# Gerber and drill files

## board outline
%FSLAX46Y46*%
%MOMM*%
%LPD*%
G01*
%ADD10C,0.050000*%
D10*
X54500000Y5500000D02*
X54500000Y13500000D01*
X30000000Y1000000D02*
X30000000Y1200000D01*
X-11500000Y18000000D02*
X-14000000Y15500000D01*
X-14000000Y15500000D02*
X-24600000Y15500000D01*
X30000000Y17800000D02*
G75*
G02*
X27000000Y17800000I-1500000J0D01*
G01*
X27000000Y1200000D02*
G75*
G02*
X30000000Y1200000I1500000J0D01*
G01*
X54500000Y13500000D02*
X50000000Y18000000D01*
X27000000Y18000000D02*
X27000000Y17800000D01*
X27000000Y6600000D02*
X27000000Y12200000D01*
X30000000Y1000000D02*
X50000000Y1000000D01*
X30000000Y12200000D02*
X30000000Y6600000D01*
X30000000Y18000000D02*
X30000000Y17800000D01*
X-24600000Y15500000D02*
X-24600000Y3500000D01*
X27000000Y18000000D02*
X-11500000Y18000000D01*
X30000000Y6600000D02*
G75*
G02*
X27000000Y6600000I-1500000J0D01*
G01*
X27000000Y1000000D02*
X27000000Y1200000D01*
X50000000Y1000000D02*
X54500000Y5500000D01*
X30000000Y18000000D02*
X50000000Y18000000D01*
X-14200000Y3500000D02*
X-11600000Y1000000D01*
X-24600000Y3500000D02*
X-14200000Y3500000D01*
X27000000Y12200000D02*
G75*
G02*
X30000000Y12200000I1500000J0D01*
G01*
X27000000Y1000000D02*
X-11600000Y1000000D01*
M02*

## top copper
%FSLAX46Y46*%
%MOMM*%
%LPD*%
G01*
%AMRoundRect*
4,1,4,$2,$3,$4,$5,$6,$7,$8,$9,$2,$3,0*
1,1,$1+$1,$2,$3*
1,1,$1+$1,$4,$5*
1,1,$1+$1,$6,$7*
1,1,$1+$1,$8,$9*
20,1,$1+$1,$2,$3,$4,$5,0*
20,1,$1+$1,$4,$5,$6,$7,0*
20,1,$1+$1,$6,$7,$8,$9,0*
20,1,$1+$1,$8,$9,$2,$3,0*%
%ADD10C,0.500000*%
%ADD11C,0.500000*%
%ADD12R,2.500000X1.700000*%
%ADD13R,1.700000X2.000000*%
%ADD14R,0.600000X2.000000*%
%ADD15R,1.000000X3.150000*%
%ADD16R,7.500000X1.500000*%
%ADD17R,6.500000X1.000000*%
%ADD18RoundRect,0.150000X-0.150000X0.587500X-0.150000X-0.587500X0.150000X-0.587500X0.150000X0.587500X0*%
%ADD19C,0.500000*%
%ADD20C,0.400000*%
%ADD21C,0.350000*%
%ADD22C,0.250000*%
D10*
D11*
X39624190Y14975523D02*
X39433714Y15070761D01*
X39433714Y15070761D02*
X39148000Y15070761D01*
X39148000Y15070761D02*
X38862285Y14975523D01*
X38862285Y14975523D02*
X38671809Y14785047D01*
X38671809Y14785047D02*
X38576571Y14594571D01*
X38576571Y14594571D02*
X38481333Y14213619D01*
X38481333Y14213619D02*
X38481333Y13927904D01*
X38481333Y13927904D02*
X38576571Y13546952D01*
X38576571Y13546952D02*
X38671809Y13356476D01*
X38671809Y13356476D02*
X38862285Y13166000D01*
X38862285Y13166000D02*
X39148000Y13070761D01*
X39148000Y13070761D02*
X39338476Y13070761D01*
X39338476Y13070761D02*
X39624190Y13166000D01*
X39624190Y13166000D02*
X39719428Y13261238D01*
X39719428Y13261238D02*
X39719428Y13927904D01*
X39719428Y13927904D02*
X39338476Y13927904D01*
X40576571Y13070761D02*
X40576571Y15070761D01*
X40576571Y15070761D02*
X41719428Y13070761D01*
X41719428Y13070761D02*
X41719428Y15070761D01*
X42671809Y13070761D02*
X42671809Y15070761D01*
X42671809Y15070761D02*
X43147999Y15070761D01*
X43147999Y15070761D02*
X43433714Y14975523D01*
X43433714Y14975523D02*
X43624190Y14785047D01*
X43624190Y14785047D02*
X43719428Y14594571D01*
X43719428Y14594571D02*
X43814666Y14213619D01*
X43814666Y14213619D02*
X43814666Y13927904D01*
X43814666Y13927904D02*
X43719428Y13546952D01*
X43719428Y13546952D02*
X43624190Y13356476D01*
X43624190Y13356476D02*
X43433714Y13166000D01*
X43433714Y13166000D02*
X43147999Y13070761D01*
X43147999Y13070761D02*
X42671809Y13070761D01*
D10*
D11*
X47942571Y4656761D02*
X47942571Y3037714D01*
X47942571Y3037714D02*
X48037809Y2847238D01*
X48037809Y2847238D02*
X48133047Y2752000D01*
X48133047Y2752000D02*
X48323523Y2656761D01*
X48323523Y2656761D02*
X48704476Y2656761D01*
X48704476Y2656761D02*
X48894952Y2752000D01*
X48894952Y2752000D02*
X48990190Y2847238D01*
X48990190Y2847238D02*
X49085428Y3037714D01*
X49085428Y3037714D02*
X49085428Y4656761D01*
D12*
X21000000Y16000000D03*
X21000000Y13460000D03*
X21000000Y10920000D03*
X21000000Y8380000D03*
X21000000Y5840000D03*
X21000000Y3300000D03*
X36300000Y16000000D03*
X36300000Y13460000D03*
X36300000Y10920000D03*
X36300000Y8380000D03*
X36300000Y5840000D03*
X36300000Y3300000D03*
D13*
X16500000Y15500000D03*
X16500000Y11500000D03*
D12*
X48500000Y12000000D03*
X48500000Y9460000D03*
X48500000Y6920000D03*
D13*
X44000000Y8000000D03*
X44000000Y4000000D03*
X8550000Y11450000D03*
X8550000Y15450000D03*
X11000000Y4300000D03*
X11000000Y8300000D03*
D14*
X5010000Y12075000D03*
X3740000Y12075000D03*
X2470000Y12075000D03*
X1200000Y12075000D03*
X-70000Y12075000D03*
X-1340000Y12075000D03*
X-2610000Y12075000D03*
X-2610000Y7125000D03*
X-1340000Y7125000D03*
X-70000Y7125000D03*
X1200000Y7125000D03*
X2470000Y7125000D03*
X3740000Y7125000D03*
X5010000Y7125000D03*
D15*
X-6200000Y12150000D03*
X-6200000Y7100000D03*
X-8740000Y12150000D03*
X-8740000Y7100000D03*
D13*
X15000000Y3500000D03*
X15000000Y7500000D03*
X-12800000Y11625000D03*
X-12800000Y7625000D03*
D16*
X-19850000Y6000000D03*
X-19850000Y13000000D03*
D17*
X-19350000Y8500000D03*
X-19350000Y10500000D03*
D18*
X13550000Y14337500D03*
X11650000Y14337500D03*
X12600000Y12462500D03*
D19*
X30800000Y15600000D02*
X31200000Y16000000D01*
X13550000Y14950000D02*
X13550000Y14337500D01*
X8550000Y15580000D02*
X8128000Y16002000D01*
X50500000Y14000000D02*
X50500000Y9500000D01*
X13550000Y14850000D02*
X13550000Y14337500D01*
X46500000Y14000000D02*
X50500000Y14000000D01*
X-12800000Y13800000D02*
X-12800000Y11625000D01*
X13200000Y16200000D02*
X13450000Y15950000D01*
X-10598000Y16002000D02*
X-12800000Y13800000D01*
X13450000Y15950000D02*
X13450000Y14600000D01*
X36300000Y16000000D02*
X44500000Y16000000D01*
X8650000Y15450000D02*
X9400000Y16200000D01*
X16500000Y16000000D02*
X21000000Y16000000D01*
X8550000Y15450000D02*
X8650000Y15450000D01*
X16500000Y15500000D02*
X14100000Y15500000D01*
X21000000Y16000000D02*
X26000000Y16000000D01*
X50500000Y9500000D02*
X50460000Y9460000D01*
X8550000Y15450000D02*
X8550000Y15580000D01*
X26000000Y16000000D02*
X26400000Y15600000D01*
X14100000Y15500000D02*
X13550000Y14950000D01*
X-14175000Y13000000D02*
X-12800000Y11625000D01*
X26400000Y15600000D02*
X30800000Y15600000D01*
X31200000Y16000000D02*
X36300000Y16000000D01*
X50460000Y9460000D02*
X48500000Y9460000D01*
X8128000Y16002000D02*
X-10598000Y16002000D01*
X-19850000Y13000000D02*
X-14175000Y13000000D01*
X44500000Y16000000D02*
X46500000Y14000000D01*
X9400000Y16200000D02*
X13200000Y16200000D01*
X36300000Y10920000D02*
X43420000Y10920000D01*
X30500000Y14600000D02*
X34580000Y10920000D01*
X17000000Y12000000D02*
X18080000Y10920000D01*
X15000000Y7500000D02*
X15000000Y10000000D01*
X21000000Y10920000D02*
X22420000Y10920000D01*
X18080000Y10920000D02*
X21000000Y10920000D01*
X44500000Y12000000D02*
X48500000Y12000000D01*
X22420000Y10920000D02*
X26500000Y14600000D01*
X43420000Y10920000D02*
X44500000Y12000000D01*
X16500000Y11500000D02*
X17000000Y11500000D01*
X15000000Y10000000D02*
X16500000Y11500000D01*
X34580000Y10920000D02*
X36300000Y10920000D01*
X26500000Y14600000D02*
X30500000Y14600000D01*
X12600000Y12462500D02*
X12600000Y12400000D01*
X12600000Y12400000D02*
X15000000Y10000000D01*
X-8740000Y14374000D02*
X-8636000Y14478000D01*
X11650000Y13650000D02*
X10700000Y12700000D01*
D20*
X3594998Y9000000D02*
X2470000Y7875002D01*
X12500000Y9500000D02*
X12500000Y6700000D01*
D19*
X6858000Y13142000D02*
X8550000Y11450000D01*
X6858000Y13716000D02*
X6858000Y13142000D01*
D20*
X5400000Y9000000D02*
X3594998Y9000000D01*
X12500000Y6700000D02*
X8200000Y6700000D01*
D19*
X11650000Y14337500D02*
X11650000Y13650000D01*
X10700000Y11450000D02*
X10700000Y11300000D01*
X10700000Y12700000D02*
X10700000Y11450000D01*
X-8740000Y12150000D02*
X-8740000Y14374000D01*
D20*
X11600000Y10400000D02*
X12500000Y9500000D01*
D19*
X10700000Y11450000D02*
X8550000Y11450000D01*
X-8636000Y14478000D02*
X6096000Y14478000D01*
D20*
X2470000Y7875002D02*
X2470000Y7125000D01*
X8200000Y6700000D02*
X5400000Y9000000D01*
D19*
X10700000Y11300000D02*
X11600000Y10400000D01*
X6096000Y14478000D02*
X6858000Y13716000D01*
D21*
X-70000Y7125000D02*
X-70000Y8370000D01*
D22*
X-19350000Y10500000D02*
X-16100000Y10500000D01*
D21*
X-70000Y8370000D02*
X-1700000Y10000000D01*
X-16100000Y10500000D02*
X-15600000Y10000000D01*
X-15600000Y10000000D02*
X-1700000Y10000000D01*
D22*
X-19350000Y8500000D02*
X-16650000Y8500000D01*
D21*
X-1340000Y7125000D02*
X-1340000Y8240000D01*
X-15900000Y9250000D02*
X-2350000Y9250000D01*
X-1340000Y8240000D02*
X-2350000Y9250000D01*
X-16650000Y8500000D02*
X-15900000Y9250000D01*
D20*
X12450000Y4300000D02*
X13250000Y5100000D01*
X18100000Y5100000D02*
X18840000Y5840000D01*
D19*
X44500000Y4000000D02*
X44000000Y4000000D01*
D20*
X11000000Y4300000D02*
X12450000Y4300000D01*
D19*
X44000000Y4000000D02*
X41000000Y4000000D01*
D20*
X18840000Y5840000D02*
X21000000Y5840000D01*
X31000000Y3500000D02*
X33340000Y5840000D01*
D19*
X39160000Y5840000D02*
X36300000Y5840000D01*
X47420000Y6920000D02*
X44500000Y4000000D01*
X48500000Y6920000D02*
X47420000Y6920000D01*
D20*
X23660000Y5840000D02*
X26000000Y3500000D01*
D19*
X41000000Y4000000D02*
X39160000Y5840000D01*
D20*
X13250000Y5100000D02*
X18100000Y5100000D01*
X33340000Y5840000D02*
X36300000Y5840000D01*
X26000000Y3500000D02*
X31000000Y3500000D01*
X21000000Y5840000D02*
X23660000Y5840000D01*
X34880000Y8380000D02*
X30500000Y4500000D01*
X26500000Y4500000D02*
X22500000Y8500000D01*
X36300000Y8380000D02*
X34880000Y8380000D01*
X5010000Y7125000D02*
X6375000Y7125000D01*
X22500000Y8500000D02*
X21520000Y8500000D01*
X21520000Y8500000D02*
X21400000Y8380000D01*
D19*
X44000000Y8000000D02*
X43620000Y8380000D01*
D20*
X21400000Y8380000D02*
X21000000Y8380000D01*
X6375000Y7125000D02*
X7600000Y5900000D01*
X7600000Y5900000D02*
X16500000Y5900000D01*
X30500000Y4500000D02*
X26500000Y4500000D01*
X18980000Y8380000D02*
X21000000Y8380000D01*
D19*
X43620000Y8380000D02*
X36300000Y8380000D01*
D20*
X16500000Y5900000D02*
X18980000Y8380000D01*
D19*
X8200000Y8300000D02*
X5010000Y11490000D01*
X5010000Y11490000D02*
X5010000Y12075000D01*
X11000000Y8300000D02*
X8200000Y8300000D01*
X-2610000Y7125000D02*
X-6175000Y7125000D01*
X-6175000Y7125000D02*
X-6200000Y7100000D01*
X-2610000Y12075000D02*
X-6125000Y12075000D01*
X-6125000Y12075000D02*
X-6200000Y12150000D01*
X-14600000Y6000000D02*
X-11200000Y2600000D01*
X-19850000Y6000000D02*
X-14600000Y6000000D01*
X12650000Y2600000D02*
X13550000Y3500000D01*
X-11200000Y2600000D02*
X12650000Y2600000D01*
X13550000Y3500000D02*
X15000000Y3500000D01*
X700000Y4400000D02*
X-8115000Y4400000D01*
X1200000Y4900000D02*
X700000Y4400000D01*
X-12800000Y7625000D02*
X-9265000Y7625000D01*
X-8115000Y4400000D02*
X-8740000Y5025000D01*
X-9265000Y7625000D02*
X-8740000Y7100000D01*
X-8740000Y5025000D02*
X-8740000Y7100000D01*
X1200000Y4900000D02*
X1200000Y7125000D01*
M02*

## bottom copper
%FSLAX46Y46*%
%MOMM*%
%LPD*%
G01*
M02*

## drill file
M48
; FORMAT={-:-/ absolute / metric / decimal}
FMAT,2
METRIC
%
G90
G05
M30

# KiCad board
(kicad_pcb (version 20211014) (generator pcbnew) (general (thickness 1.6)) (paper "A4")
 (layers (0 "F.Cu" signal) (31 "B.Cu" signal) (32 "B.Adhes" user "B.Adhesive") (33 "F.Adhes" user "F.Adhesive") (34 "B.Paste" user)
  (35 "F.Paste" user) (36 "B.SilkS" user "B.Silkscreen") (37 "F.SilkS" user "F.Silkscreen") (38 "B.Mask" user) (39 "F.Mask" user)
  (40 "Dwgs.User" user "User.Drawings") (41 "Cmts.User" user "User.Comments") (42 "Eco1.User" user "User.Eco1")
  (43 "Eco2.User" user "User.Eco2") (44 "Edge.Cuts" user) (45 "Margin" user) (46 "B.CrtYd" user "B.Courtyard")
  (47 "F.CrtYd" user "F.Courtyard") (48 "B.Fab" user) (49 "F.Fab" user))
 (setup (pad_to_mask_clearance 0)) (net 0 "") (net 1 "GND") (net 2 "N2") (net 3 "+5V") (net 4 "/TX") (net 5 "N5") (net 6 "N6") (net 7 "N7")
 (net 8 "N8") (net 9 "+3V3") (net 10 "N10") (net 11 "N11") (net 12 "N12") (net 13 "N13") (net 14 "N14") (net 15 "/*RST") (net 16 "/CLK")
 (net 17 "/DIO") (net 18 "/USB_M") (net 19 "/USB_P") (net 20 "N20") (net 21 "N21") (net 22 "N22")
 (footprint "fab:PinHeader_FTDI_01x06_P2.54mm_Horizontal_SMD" (layer "F.Cu") (at 21 -16)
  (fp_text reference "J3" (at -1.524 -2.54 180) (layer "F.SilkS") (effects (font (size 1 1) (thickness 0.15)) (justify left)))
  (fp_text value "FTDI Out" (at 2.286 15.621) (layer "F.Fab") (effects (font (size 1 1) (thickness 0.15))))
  (pad "2" smd rect locked (at 0 0) (size 2.5 1.7) (layers "F.Cu" "F.Paste" "F.Mask") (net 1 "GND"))
  (pad "1" smd rect locked (at 0 2.54) (size 2.5 1.7) (layers "F.Cu" "F.Paste" "F.Mask") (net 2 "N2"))
  (pad "3" smd rect locked (at 0 5.08) (size 2.5 1.7) (layers "F.Cu" "F.Paste" "F.Mask") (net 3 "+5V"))
  (pad "4" smd rect locked (at 0 7.62) (size 2.5 1.7) (layers "F.Cu" "F.Paste" "F.Mask") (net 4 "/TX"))
  (pad "5" smd rect locked (at 0 10.16) (size 2.5 1.7) (layers "F.Cu" "F.Paste" "F.Mask") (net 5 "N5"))
  (pad "6" smd rect locked (at 0 12.7) (size 2.5 1.7) (layers "F.Cu" "F.Paste" "F.Mask") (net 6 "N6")))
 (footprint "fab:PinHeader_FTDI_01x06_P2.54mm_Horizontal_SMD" (layer "F.Cu") (at 36.3 -16)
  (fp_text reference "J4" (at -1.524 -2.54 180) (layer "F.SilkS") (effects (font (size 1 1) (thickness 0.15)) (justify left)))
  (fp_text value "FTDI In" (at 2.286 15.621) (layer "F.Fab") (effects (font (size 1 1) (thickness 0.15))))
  (pad "1" smd rect locked (at 0 0) (size 2.5 1.7) (layers "F.Cu" "F.Paste" "F.Mask") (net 1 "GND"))
  (pad "2" smd rect locked (at 0 2.54) (size 2.5 1.7) (layers "F.Cu" "F.Paste" "F.Mask") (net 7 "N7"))
  (pad "3" smd rect locked (at 0 5.08) (size 2.5 1.7) (layers "F.Cu" "F.Paste" "F.Mask") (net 3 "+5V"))
  (pad "4" smd rect locked (at 0 7.62) (size 2.5 1.7) (layers "F.Cu" "F.Paste" "F.Mask") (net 4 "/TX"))
  (pad "5" smd rect locked (at 0 10.16) (size 2.5 1.7) (layers "F.Cu" "F.Paste" "F.Mask") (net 5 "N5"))
  (pad "6" smd rect locked (at 0 12.7) (size 2.5 1.7) (layers "F.Cu" "F.Paste" "F.Mask") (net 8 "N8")))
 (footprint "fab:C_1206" (layer "F.Cu") (at 16.5 -13.5 -90)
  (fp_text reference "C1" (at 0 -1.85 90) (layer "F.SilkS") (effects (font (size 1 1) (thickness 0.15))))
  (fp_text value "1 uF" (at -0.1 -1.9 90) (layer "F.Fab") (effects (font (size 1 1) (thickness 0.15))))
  (pad "1" smd rect locked (at -2 0 270) (size 2 1.7) (layers "F.Cu" "F.Paste" "F.Mask") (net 1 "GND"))
  (pad "2" smd rect locked (at 2 0 270) (size 2 1.7) (layers "F.Cu" "F.Paste" "F.Mask") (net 3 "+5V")))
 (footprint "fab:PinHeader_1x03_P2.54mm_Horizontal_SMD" (layer "F.Cu") (at 48.5 -12)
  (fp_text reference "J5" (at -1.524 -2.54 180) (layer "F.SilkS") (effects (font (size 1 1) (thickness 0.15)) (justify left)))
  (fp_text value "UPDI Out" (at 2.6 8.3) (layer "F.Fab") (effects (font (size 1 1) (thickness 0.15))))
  (pad "1" smd rect locked (at 0 0) (size 2.5 1.7) (layers "F.Cu" "F.Paste" "F.Mask") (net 3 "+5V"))
  (pad "2" smd rect locked (at 0 2.54) (size 2.5 1.7) (layers "F.Cu" "F.Paste" "F.Mask") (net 1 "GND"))
  (pad "3" smd rect locked (at 0 5.08) (size 2.5 1.7) (layers "F.Cu" "F.Paste" "F.Mask") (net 5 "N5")))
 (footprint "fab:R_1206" (layer "F.Cu") (at 44 -6 -90)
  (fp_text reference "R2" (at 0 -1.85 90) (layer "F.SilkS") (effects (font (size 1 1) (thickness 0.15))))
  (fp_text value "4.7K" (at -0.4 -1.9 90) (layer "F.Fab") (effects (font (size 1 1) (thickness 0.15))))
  (pad "1" smd rect locked (at -2 0 270) (size 2 1.7) (layers "F.Cu" "F.Paste" "F.Mask") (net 4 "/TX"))
  (pad "2" smd rect locked (at 2 0 270) (size 2 1.7) (layers "F.Cu" "F.Paste" "F.Mask") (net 5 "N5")))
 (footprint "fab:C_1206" (layer "F.Cu") (at 8.55 -13.45 90)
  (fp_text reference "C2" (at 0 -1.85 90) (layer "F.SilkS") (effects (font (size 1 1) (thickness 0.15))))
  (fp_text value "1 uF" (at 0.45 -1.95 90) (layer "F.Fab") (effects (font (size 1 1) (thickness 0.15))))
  (pad "1" smd rect locked (at -2 0 90) (size 2 1.7) (layers "F.Cu" "F.Paste" "F.Mask") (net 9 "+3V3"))
  (pad "2" smd rect locked (at 2 0 90) (size 2 1.7) (layers "F.Cu" "F.Paste" "F.Mask") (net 1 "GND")))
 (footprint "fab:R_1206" (layer "F.Cu") (at 11 -6.3 90)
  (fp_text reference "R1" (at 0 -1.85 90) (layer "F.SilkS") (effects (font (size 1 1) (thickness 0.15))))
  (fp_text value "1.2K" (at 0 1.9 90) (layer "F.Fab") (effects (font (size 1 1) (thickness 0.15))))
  (pad "1" smd rect locked (at -2 0 90) (size 2 1.7) (layers "F.Cu" "F.Paste" "F.Mask") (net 5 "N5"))
  (pad "2" smd rect locked (at 2 0 90) (size 2 1.7) (layers "F.Cu" "F.Paste" "F.Mask") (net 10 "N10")))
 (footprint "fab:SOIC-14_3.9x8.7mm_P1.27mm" (layer "F.Cu") (at 1.2 -9.6 -90)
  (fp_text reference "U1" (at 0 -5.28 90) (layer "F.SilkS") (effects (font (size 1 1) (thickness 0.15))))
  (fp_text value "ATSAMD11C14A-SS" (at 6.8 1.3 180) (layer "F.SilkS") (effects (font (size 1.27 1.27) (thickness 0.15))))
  (pad "1" smd rect locked (at -2.475 -3.81 270) (size 2 0.6) (layers "F.Cu" "F.Paste" "F.Mask") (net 10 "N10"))
  (pad "2" smd rect locked (at -2.475 -2.54 270) (size 2 0.6) (layers "F.Cu" "F.Paste" "F.Mask") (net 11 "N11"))
  (pad "3" smd rect locked (at -2.475 -1.27 270) (size 2 0.6) (layers "F.Cu" "F.Paste" "F.Mask") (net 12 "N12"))
  (pad "4" smd rect locked (at -2.475 0 270) (size 2 0.6) (layers "F.Cu" "F.Paste" "F.Mask") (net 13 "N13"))
  (pad "5" smd rect locked (at -2.475 1.27 270) (size 2 0.6) (layers "F.Cu" "F.Paste" "F.Mask") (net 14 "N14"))
  (pad "6" smd rect locked (at -2.475 2.54 270) (size 2 0.6) (layers "F.Cu" "F.Paste" "F.Mask") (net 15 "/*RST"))
  (pad "7" smd rect locked (at -2.475 3.81 270) (size 2 0.6) (layers "F.Cu" "F.Paste" "F.Mask") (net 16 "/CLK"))
  (pad "8" smd rect locked (at 2.475 3.81 270) (size 2 0.6) (layers "F.Cu" "F.Paste" "F.Mask") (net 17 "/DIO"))
  (pad "9" smd rect locked (at 2.475 2.54 270) (size 2 0.6) (layers "F.Cu" "F.Paste" "F.Mask") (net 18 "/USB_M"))
  (pad "10" smd rect locked (at 2.475 1.27 270) (size 2 0.6) (layers "F.Cu" "F.Paste" "F.Mask") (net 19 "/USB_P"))
  (pad "11" smd rect locked (at 2.475 0 270) (size 2 0.6) (layers "F.Cu" "F.Paste" "F.Mask") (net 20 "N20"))
  (pad "12" smd rect locked (at 2.475 -1.27 270) (size 2 0.6) (layers "F.Cu" "F.Paste" "F.Mask") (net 9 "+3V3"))
  (pad "13" smd rect locked (at 2.475 -2.54 270) (size 2 0.6) (layers "F.Cu" "F.Paste" "F.Mask") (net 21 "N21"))
  (pad "14" smd rect locked (at 2.475 -3.81 270) (size 2 0.6) (layers "F.Cu" "F.Paste" "F.Mask") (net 4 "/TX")))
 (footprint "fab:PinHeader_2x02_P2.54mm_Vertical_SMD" (layer "F.Cu") (at -7.47 -9.625 -90)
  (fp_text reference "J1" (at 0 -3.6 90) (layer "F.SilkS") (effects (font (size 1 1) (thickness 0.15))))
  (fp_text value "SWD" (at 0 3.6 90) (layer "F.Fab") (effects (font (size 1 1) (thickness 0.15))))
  (pad "1" smd rect locked (at -2.525 -1.27 270) (size 3.15 1) (layers "F.Cu" "F.Paste" "F.Mask") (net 16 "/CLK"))
  (pad "2" smd rect locked (at 2.525 -1.27 270) (size 3.15 1) (layers "F.Cu" "F.Paste" "F.Mask") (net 17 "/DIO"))
  (pad "3" smd rect locked (at -2.525 1.27 270) (size 3.15 1) (layers "F.Cu" "F.Paste" "F.Mask") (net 9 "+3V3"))
  (pad "4" smd rect locked (at 2.525 1.27 270) (size 3.15 1) (layers "F.Cu" "F.Paste" "F.Mask") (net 20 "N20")))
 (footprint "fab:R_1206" (layer "F.Cu") (at 15 -5.5 90)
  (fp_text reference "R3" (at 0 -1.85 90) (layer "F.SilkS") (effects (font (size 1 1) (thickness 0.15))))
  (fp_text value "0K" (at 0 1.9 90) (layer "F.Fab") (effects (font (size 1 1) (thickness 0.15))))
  (pad "1" smd rect locked (at -2 0 90) (size 2 1.7) (layers "F.Cu" "F.Paste" "F.Mask") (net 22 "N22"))
  (pad "2" smd rect locked (at 2 0 90) (size 2 1.7) (layers "F.Cu" "F.Paste" "F.Mask") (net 3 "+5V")))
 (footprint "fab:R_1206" (layer "F.Cu") (at -12.8 -9.625 -90)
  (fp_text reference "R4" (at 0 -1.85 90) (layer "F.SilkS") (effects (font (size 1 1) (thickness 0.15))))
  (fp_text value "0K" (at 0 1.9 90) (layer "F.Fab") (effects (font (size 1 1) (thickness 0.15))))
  (pad "1" smd rect locked (at -2 0 270) (size 2 1.7) (layers "F.Cu" "F.Paste" "F.Mask") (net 1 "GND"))
  (pad "2" smd rect locked (at 2 0 270) (size 2 1.7) (layers "F.Cu" "F.Paste" "F.Mask") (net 20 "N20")))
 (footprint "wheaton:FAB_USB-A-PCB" (layer "F.Cu") (at -19.65 -9.5)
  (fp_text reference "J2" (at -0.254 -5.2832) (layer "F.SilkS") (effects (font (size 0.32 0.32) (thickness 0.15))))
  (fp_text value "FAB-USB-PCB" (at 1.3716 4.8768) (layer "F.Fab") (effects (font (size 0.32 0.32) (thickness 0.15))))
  (pad "5V" smd rect locked (at -0.2 3.5) (size 7.5 1.5) (layers "F.Cu" "F.Paste" "F.Mask") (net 22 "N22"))
  (pad "GND" smd rect locked (at -0.2 -3.5) (size 7.5 1.5) (layers "F.Cu" "F.Paste" "F.Mask") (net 1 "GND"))
  (pad "USB_M" smd rect locked (at 0.3 1) (size 6.5 1) (layers "F.Cu" "F.Paste" "F.Mask") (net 18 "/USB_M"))
  (pad "USB_P" smd rect locked (at 0.3 -1) (size 6.5 1) (layers "F.Cu" "F.Paste" "F.Mask") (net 19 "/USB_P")))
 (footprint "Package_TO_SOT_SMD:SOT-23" (layer "F.Cu") (at 12.6 -13.4 -90)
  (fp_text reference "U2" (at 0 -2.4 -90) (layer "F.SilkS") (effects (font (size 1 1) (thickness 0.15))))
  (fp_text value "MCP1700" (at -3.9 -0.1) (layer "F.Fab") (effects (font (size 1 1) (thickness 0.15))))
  (pad "1" smd roundrect (at -0.9375 -0.95 270) (size 1.475 0.6) (layers "F.Cu" "F.Paste" "F.Mask") (roundrect_rratio 0.25) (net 1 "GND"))
  (pad "2" smd roundrect (at -0.9375 0.95 270) (size 1.475 0.6) (layers "F.Cu" "F.Paste" "F.Mask") (roundrect_rratio 0.25) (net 9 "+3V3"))
  (pad "3" smd roundrect (at 0.9375 0 270) (size 1.475 0.6) (layers "F.Cu" "F.Paste" "F.Mask") (roundrect_rratio 0.25) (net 3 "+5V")))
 (gr_line (start 54.5 -5.5) (end 54.5 -13.5) (layer "Edge.Cuts") (width 0.05))
 (gr_line (start 30 -1) (end 30 -1.2) (layer "Edge.Cuts") (width 0.05))
 (gr_line (start -11.5 -18) (end -14 -15.5) (layer "Edge.Cuts") (width 0.05))
 (gr_line (start -14 -15.5) (end -24.6 -15.5) (layer "Edge.Cuts") (width 0.05))
 (gr_arc (start 30 -17.8) (mid 28.5 -16.3) (end 27 -17.8) (layer "Edge.Cuts") (width 0.05))
 (gr_arc (start 27 -1.2) (mid 28.5 -2.7) (end 30 -1.2) (layer "Edge.Cuts") (width 0.05))
 (gr_line (start 54.5 -13.5) (end 50 -18) (layer "Edge.Cuts") (width 0.05))
 (gr_line (start 27 -18) (end 27 -17.8) (layer "Edge.Cuts") (width 0.05))
 (gr_line (start 27 -6.6) (end 27 -12.2) (layer "Edge.Cuts") (width 0.05))
 (gr_line (start 30 -1) (end 50 -1) (layer "Edge.Cuts") (width 0.05))
 (gr_line (start 30 -12.2) (end 30 -6.6) (layer "Edge.Cuts") (width 0.05))
 (gr_line (start 30 -18) (end 30 -17.8) (layer "Edge.Cuts") (width 0.05))
 (gr_line (start -24.6 -15.5) (end -24.6 -3.5) (layer "Edge.Cuts") (width 0.05))
 (gr_line (start 27 -18) (end -11.5 -18) (layer "Edge.Cuts") (width 0.05))
 (gr_arc (start 30 -6.6) (mid 28.5 -5.1) (end 27 -6.6) (layer "Edge.Cuts") (width 0.05))
 (gr_line (start 27 -1) (end 27 -1.2) (layer "Edge.Cuts") (width 0.05))
 (gr_line (start 50 -1) (end 54.5 -5.5) (layer "Edge.Cuts") (width 0.05))
 (gr_line (start 30 -18) (end 50 -18) (layer "Edge.Cuts") (width 0.05))
 (gr_line (start -14.2 -3.5) (end -11.6 -1) (layer "Edge.Cuts") (width 0.05))
 (gr_line (start -24.6 -3.5) (end -14.2 -3.5) (layer "Edge.Cuts") (width 0.05))
 (gr_arc (start 27 -12.2) (mid 28.5 -13.7) (end 30 -12.2) (layer "Edge.Cuts") (width 0.05))
 (gr_line (start 27 -1) (end -11.6 -1) (layer "Edge.Cuts") (width 0.05))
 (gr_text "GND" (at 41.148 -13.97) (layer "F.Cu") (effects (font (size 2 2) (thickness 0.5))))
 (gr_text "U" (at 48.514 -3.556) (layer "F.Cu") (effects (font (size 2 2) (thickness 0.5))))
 (segment (start 30.8 -15.6) (end 31.2 -16) (width 0.5) (layer "F.Cu") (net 1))
 (segment (start 13.55 -14.95) (end 13.55 -14.3375) (width 0.5) (layer "F.Cu") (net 1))
 (segment (start 8.55 -15.58) (end 8.128 -16.002) (width 0.5) (layer "F.Cu") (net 1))
 (segment (start 50.5 -14) (end 50.5 -9.5) (width 0.5) (layer "F.Cu") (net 1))
 (segment (start 13.55 -14.85) (end 13.55 -14.3375) (width 0.5) (layer "F.Cu") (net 1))
 (segment (start 46.5 -14) (end 50.5 -14) (width 0.5) (layer "F.Cu") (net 1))
 (segment (start -12.8 -13.8) (end -12.8 -11.625) (width 0.5) (layer "F.Cu") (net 1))
 (segment (start 13.2 -16.2) (end 13.45 -15.95) (width 0.5) (layer "F.Cu") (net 1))
 (segment (start -10.598 -16.002) (end -12.8 -13.8) (width 0.5) (layer "F.Cu") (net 1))
 (segment (start 13.45 -15.95) (end 13.45 -14.6) (width 0.5) (layer "F.Cu") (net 1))
 (segment (start 36.3 -16) (end 44.5 -16) (width 0.5) (layer "F.Cu") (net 1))
 (segment (start 8.65 -15.45) (end 9.4 -16.2) (width 0.5) (layer "F.Cu") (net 1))
 (segment (start 16.5 -16) (end 21 -16) (width 0.5) (layer "F.Cu") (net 1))
 (segment (start 8.55 -15.45) (end 8.65 -15.45) (width 0.5) (layer "F.Cu") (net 1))
 (segment (start 16.5 -15.5) (end 14.1 -15.5) (width 0.5) (layer "F.Cu") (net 1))
 (segment (start 21 -16) (end 26 -16) (width 0.5) (layer "F.Cu") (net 1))
 (segment (start 50.5 -9.5) (end 50.46 -9.46) (width 0.5) (layer "F.Cu") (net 1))
 (segment (start 8.55 -15.45) (end 8.55 -15.58) (width 0.5) (layer "F.Cu") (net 1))
 (segment (start 26 -16) (end 26.4 -15.6) (width 0.5) (layer "F.Cu") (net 1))
 (segment (start 14.1 -15.5) (end 13.55 -14.95) (width 0.5) (layer "F.Cu") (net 1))
 (segment (start -14.175 -13) (end -12.8 -11.625) (width 0.5) (layer "F.Cu") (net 1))
 (segment (start 26.4 -15.6) (end 30.8 -15.6) (width 0.5) (layer "F.Cu") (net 1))
 (segment (start 31.2 -16) (end 36.3 -16) (width 0.5) (layer "F.Cu") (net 1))
 (segment (start 50.46 -9.46) (end 48.5 -9.46) (width 0.5) (layer "F.Cu") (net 1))
 (segment (start 8.128 -16.002) (end -10.598 -16.002) (width 0.5) (layer "F.Cu") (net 1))
 (segment (start -19.85 -13) (end -14.175 -13) (width 0.5) (layer "F.Cu") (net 1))
 (segment (start 44.5 -16) (end 46.5 -14) (width 0.5) (layer "F.Cu") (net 1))
 (segment (start 9.4 -16.2) (end 13.2 -16.2) (width 0.5) (layer "F.Cu") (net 1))
 (segment (start 36.3 -10.92) (end 43.42 -10.92) (width 0.5) (layer "F.Cu") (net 3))
 (segment (start 30.5 -14.6) (end 34.58 -10.92) (width 0.5) (layer "F.Cu") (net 3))
 (segment (start 17 -12) (end 18.08 -10.92) (width 0.5) (layer "F.Cu") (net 3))
 (segment (start 15 -7.5) (end 15 -10) (width 0.5) (layer "F.Cu") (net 3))
 (segment (start 21 -10.92) (end 22.42 -10.92) (width 0.5) (layer "F.Cu") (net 3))
 (segment (start 18.08 -10.92) (end 21 -10.92) (width 0.5) (layer "F.Cu") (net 3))
 (segment (start 44.5 -12) (end 48.5 -12) (width 0.5) (layer "F.Cu") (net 3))
 (segment (start 22.42 -10.92) (end 26.5 -14.6) (width 0.5) (layer "F.Cu") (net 3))
 (segment (start 43.42 -10.92) (end 44.5 -12) (width 0.5) (layer "F.Cu") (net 3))
 (segment (start 16.5 -11.5) (end 17 -11.5) (width 0.5) (layer "F.Cu") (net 3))
 (segment (start 15 -10) (end 16.5 -11.5) (width 0.5) (layer "F.Cu") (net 3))
 (segment (start 34.58 -10.92) (end 36.3 -10.92) (width 0.5) (layer "F.Cu") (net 3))
 (segment (start 26.5 -14.6) (end 30.5 -14.6) (width 0.5) (layer "F.Cu") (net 3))
 (segment (start 12.6 -12.4625) (end 12.6 -12.4) (width 0.5) (layer "F.Cu") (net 3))
 (segment (start 12.6 -12.4) (end 15 -10) (width 0.5) (layer "F.Cu") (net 3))
 (segment (start -8.74 -14.374) (end -8.636 -14.478) (width 0.5) (layer "F.Cu") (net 9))
 (segment (start 11.65 -13.65) (end 10.7 -12.7) (width 0.5) (layer "F.Cu") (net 9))
 (segment (start 3.594998 -9) (end 2.47 -7.875002) (width 0.4) (layer "F.Cu") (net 9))
 (segment (start 12.5 -9.5) (end 12.5 -6.7) (width 0.4) (layer "F.Cu") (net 9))
 (segment (start 6.858 -13.142) (end 8.55 -11.45) (width 0.5) (layer "F.Cu") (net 9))
 (segment (start 6.858 -13.716) (end 6.858 -13.142) (width 0.5) (layer "F.Cu") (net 9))
 (segment (start 5.4 -9) (end 3.594998 -9) (width 0.4) (layer "F.Cu") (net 9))
 (segment (start 12.5 -6.7) (end 8.2 -6.7) (width 0.4) (layer "F.Cu") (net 9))
 (segment (start 11.65 -14.3375) (end 11.65 -13.65) (width 0.5) (layer "F.Cu") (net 9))
 (segment (start 10.7 -11.45) (end 10.7 -11.3) (width 0.5) (layer "F.Cu") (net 9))
 (segment (start 10.7 -12.7) (end 10.7 -11.45) (width 0.5) (layer "F.Cu") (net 9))
 (segment (start -8.74 -12.15) (end -8.74 -14.374) (width 0.5) (layer "F.Cu") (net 9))
 (segment (start 11.6 -10.4) (end 12.5 -9.5) (width 0.4) (layer "F.Cu") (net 9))
 (segment (start 10.7 -11.45) (end 8.55 -11.45) (width 0.5) (layer "F.Cu") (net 9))
 (segment (start -8.636 -14.478) (end 6.096 -14.478) (width 0.5) (layer "F.Cu") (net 9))
 (segment (start 2.47 -7.875002) (end 2.47 -7.125) (width 0.4) (layer "F.Cu") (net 9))
 (segment (start 8.2 -6.7) (end 5.4 -9) (width 0.4) (layer "F.Cu") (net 9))
 (segment (start 10.7 -11.3) (end 11.6 -10.4) (width 0.5) (layer "F.Cu") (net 9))
 (segment (start 6.096 -14.478) (end 6.858 -13.716) (width 0.5) (layer "F.Cu") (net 9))
 (segment (start -0.07 -7.125) (end -0.07 -8.37) (width 0.35) (layer "F.Cu") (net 19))
 (segment (start -19.35 -10.5) (end -16.1 -10.5) (width 0.25) (layer "F.Cu") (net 19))
 (segment (start -0.07 -8.37) (end -1.7 -10) (width 0.35) (layer "F.Cu") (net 19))
 (segment (start -16.1 -10.5) (end -15.6 -10) (width 0.35) (layer "F.Cu") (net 19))
 (segment (start -15.6 -10) (end -1.7 -10) (width 0.35) (layer "F.Cu") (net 19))
 (segment (start -19.35 -8.5) (end -16.65 -8.5) (width 0.25) (layer "F.Cu") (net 18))
 (segment (start -1.34 -7.125) (end -1.34 -8.24) (width 0.35) (layer "F.Cu") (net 18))
 (segment (start -15.9 -9.25) (end -2.35 -9.25) (width 0.35) (layer "F.Cu") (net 18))
 (segment (start -1.34 -8.24) (end -2.35 -9.25) (width 0.35) (layer "F.Cu") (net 18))
 (segment (start -16.65 -8.5) (end -15.9 -9.25) (width 0.35) (layer "F.Cu") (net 18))
 (segment (start 12.45 -4.3) (end 13.25 -5.1) (width 0.4) (layer "F.Cu") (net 5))
 (segment (start 18.1 -5.1) (end 18.84 -5.84) (width 0.4) (layer "F.Cu") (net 5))
 (segment (start 44.5 -4) (end 44 -4) (width 0.5) (layer "F.Cu") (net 5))
 (segment (start 11 -4.3) (end 12.45 -4.3) (width 0.4) (layer "F.Cu") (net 5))
 (segment (start 44 -4) (end 41 -4) (width 0.5) (layer "F.Cu") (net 5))
 (segment (start 18.84 -5.84) (end 21 -5.84) (width 0.4) (layer "F.Cu") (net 5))
 (segment (start 31 -3.5) (end 33.34 -5.84) (width 0.4) (layer "F.Cu") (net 5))
 (segment (start 39.16 -5.84) (end 36.3 -5.84) (width 0.5) (layer "F.Cu") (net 5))
 (segment (start 47.42 -6.92) (end 44.5 -4) (width 0.5) (layer "F.Cu") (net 5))
 (segment (start 48.5 -6.92) (end 47.42 -6.92) (width 0.5) (layer "F.Cu") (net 5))
 (segment (start 23.66 -5.84) (end 26 -3.5) (width 0.4) (layer "F.Cu") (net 5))
 (segment (start 41 -4) (end 39.16 -5.84) (width 0.5) (layer "F.Cu") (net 5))
 (segment (start 13.25 -5.1) (end 18.1 -5.1) (width 0.4) (layer "F.Cu") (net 5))
 (segment (start 33.34 -5.84) (end 36.3 -5.84) (width 0.4) (layer "F.Cu") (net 5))
 (segment (start 26 -3.5) (end 31 -3.5) (width 0.4) (layer "F.Cu") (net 5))
 (segment (start 21 -5.84) (end 23.66 -5.84) (width 0.4) (layer "F.Cu") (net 5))
 (segment (start 34.88 -8.38) (end 30.5 -4.5) (width 0.4) (layer "F.Cu") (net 4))
 (segment (start 26.5 -4.5) (end 22.5 -8.5) (width 0.4) (layer "F.Cu") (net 4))
 (segment (start 36.3 -8.38) (end 34.88 -8.38) (width 0.4) (layer "F.Cu") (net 4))
 (segment (start 5.01 -7.125) (end 6.375 -7.125) (width 0.4) (layer "F.Cu") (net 4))
 (segment (start 22.5 -8.5) (end 21.52 -8.5) (width 0.4) (layer "F.Cu") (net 4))
 (segment (start 21.52 -8.5) (end 21.4 -8.38) (width 0.4) (layer "F.Cu") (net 4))
 (segment (start 44 -8) (end 43.62 -8.38) (width 0.5) (layer "F.Cu") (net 4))
 (segment (start 21.4 -8.38) (end 21 -8.38) (width 0.4) (layer "F.Cu") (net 4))
 (segment (start 6.375 -7.125) (end 7.6 -5.9) (width 0.4) (layer "F.Cu") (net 4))
 (segment (start 7.6 -5.9) (end 16.5 -5.9) (width 0.4) (layer "F.Cu") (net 4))
 (segment (start 30.5 -4.5) (end 26.5 -4.5) (width 0.4) (layer "F.Cu") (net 4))
 (segment (start 18.98 -8.38) (end 21 -8.38) (width 0.4) (layer "F.Cu") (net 4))
 (segment (start 43.62 -8.38) (end 36.3 -8.38) (width 0.5) (layer "F.Cu") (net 4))
 (segment (start 16.5 -5.9) (end 18.98 -8.38) (width 0.4) (layer "F.Cu") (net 4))
 (segment (start 8.2 -8.3) (end 5.01 -11.49) (width 0.5) (layer "F.Cu") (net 10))
 (segment (start 5.01 -11.49) (end 5.01 -12.075) (width 0.5) (layer "F.Cu") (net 10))
 (segment (start 11 -8.3) (end 8.2 -8.3) (width 0.5) (layer "F.Cu") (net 10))
 (segment (start -2.61 -7.125) (end -6.175 -7.125) (width 0.5) (layer "F.Cu") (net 17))
 (segment (start -6.175 -7.125) (end -6.2 -7.1) (width 0.5) (layer "F.Cu") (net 17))
 (segment (start -2.61 -12.075) (end -6.125 -12.075) (width 0.5) (layer "F.Cu") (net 16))
 (segment (start -6.125 -12.075) (end -6.2 -12.15) (width 0.5) (layer "F.Cu") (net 16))
 (segment (start -14.6 -6) (end -11.2 -2.6) (width 0.5) (layer "F.Cu") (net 22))
 (segment (start -19.85 -6) (end -14.6 -6) (width 0.5) (layer "F.Cu") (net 22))
 (segment (start 12.65 -2.6) (end 13.55 -3.5) (width 0.5) (layer "F.Cu") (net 22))
 (segment (start -11.2 -2.6) (end 12.65 -2.6) (width 0.5) (layer "F.Cu") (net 22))
 (segment (start 13.55 -3.5) (end 15 -3.5) (width 0.5) (layer "F.Cu") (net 22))
 (segment (start 0.7 -4.4) (end -8.115 -4.4) (width 0.5) (layer "F.Cu") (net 20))
 (segment (start 1.2 -4.9) (end 0.7 -4.4) (width 0.5) (layer "F.Cu") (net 20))
 (segment (start -12.8 -7.625) (end -9.265 -7.625) (width 0.5) (layer "F.Cu") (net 20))
 (segment (start -8.115 -4.4) (end -8.74 -5.025) (width 0.5) (layer "F.Cu") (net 20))
 (segment (start -9.265 -7.625) (end -8.74 -7.1) (width 0.5) (layer "F.Cu") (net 20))
 (segment (start -8.74 -5.025) (end -8.74 -7.1) (width 0.5) (layer "F.Cu") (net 20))
 (segment (start 1.2 -4.9) (end 1.2 -7.125) (width 0.5) (layer "F.Cu") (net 20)))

